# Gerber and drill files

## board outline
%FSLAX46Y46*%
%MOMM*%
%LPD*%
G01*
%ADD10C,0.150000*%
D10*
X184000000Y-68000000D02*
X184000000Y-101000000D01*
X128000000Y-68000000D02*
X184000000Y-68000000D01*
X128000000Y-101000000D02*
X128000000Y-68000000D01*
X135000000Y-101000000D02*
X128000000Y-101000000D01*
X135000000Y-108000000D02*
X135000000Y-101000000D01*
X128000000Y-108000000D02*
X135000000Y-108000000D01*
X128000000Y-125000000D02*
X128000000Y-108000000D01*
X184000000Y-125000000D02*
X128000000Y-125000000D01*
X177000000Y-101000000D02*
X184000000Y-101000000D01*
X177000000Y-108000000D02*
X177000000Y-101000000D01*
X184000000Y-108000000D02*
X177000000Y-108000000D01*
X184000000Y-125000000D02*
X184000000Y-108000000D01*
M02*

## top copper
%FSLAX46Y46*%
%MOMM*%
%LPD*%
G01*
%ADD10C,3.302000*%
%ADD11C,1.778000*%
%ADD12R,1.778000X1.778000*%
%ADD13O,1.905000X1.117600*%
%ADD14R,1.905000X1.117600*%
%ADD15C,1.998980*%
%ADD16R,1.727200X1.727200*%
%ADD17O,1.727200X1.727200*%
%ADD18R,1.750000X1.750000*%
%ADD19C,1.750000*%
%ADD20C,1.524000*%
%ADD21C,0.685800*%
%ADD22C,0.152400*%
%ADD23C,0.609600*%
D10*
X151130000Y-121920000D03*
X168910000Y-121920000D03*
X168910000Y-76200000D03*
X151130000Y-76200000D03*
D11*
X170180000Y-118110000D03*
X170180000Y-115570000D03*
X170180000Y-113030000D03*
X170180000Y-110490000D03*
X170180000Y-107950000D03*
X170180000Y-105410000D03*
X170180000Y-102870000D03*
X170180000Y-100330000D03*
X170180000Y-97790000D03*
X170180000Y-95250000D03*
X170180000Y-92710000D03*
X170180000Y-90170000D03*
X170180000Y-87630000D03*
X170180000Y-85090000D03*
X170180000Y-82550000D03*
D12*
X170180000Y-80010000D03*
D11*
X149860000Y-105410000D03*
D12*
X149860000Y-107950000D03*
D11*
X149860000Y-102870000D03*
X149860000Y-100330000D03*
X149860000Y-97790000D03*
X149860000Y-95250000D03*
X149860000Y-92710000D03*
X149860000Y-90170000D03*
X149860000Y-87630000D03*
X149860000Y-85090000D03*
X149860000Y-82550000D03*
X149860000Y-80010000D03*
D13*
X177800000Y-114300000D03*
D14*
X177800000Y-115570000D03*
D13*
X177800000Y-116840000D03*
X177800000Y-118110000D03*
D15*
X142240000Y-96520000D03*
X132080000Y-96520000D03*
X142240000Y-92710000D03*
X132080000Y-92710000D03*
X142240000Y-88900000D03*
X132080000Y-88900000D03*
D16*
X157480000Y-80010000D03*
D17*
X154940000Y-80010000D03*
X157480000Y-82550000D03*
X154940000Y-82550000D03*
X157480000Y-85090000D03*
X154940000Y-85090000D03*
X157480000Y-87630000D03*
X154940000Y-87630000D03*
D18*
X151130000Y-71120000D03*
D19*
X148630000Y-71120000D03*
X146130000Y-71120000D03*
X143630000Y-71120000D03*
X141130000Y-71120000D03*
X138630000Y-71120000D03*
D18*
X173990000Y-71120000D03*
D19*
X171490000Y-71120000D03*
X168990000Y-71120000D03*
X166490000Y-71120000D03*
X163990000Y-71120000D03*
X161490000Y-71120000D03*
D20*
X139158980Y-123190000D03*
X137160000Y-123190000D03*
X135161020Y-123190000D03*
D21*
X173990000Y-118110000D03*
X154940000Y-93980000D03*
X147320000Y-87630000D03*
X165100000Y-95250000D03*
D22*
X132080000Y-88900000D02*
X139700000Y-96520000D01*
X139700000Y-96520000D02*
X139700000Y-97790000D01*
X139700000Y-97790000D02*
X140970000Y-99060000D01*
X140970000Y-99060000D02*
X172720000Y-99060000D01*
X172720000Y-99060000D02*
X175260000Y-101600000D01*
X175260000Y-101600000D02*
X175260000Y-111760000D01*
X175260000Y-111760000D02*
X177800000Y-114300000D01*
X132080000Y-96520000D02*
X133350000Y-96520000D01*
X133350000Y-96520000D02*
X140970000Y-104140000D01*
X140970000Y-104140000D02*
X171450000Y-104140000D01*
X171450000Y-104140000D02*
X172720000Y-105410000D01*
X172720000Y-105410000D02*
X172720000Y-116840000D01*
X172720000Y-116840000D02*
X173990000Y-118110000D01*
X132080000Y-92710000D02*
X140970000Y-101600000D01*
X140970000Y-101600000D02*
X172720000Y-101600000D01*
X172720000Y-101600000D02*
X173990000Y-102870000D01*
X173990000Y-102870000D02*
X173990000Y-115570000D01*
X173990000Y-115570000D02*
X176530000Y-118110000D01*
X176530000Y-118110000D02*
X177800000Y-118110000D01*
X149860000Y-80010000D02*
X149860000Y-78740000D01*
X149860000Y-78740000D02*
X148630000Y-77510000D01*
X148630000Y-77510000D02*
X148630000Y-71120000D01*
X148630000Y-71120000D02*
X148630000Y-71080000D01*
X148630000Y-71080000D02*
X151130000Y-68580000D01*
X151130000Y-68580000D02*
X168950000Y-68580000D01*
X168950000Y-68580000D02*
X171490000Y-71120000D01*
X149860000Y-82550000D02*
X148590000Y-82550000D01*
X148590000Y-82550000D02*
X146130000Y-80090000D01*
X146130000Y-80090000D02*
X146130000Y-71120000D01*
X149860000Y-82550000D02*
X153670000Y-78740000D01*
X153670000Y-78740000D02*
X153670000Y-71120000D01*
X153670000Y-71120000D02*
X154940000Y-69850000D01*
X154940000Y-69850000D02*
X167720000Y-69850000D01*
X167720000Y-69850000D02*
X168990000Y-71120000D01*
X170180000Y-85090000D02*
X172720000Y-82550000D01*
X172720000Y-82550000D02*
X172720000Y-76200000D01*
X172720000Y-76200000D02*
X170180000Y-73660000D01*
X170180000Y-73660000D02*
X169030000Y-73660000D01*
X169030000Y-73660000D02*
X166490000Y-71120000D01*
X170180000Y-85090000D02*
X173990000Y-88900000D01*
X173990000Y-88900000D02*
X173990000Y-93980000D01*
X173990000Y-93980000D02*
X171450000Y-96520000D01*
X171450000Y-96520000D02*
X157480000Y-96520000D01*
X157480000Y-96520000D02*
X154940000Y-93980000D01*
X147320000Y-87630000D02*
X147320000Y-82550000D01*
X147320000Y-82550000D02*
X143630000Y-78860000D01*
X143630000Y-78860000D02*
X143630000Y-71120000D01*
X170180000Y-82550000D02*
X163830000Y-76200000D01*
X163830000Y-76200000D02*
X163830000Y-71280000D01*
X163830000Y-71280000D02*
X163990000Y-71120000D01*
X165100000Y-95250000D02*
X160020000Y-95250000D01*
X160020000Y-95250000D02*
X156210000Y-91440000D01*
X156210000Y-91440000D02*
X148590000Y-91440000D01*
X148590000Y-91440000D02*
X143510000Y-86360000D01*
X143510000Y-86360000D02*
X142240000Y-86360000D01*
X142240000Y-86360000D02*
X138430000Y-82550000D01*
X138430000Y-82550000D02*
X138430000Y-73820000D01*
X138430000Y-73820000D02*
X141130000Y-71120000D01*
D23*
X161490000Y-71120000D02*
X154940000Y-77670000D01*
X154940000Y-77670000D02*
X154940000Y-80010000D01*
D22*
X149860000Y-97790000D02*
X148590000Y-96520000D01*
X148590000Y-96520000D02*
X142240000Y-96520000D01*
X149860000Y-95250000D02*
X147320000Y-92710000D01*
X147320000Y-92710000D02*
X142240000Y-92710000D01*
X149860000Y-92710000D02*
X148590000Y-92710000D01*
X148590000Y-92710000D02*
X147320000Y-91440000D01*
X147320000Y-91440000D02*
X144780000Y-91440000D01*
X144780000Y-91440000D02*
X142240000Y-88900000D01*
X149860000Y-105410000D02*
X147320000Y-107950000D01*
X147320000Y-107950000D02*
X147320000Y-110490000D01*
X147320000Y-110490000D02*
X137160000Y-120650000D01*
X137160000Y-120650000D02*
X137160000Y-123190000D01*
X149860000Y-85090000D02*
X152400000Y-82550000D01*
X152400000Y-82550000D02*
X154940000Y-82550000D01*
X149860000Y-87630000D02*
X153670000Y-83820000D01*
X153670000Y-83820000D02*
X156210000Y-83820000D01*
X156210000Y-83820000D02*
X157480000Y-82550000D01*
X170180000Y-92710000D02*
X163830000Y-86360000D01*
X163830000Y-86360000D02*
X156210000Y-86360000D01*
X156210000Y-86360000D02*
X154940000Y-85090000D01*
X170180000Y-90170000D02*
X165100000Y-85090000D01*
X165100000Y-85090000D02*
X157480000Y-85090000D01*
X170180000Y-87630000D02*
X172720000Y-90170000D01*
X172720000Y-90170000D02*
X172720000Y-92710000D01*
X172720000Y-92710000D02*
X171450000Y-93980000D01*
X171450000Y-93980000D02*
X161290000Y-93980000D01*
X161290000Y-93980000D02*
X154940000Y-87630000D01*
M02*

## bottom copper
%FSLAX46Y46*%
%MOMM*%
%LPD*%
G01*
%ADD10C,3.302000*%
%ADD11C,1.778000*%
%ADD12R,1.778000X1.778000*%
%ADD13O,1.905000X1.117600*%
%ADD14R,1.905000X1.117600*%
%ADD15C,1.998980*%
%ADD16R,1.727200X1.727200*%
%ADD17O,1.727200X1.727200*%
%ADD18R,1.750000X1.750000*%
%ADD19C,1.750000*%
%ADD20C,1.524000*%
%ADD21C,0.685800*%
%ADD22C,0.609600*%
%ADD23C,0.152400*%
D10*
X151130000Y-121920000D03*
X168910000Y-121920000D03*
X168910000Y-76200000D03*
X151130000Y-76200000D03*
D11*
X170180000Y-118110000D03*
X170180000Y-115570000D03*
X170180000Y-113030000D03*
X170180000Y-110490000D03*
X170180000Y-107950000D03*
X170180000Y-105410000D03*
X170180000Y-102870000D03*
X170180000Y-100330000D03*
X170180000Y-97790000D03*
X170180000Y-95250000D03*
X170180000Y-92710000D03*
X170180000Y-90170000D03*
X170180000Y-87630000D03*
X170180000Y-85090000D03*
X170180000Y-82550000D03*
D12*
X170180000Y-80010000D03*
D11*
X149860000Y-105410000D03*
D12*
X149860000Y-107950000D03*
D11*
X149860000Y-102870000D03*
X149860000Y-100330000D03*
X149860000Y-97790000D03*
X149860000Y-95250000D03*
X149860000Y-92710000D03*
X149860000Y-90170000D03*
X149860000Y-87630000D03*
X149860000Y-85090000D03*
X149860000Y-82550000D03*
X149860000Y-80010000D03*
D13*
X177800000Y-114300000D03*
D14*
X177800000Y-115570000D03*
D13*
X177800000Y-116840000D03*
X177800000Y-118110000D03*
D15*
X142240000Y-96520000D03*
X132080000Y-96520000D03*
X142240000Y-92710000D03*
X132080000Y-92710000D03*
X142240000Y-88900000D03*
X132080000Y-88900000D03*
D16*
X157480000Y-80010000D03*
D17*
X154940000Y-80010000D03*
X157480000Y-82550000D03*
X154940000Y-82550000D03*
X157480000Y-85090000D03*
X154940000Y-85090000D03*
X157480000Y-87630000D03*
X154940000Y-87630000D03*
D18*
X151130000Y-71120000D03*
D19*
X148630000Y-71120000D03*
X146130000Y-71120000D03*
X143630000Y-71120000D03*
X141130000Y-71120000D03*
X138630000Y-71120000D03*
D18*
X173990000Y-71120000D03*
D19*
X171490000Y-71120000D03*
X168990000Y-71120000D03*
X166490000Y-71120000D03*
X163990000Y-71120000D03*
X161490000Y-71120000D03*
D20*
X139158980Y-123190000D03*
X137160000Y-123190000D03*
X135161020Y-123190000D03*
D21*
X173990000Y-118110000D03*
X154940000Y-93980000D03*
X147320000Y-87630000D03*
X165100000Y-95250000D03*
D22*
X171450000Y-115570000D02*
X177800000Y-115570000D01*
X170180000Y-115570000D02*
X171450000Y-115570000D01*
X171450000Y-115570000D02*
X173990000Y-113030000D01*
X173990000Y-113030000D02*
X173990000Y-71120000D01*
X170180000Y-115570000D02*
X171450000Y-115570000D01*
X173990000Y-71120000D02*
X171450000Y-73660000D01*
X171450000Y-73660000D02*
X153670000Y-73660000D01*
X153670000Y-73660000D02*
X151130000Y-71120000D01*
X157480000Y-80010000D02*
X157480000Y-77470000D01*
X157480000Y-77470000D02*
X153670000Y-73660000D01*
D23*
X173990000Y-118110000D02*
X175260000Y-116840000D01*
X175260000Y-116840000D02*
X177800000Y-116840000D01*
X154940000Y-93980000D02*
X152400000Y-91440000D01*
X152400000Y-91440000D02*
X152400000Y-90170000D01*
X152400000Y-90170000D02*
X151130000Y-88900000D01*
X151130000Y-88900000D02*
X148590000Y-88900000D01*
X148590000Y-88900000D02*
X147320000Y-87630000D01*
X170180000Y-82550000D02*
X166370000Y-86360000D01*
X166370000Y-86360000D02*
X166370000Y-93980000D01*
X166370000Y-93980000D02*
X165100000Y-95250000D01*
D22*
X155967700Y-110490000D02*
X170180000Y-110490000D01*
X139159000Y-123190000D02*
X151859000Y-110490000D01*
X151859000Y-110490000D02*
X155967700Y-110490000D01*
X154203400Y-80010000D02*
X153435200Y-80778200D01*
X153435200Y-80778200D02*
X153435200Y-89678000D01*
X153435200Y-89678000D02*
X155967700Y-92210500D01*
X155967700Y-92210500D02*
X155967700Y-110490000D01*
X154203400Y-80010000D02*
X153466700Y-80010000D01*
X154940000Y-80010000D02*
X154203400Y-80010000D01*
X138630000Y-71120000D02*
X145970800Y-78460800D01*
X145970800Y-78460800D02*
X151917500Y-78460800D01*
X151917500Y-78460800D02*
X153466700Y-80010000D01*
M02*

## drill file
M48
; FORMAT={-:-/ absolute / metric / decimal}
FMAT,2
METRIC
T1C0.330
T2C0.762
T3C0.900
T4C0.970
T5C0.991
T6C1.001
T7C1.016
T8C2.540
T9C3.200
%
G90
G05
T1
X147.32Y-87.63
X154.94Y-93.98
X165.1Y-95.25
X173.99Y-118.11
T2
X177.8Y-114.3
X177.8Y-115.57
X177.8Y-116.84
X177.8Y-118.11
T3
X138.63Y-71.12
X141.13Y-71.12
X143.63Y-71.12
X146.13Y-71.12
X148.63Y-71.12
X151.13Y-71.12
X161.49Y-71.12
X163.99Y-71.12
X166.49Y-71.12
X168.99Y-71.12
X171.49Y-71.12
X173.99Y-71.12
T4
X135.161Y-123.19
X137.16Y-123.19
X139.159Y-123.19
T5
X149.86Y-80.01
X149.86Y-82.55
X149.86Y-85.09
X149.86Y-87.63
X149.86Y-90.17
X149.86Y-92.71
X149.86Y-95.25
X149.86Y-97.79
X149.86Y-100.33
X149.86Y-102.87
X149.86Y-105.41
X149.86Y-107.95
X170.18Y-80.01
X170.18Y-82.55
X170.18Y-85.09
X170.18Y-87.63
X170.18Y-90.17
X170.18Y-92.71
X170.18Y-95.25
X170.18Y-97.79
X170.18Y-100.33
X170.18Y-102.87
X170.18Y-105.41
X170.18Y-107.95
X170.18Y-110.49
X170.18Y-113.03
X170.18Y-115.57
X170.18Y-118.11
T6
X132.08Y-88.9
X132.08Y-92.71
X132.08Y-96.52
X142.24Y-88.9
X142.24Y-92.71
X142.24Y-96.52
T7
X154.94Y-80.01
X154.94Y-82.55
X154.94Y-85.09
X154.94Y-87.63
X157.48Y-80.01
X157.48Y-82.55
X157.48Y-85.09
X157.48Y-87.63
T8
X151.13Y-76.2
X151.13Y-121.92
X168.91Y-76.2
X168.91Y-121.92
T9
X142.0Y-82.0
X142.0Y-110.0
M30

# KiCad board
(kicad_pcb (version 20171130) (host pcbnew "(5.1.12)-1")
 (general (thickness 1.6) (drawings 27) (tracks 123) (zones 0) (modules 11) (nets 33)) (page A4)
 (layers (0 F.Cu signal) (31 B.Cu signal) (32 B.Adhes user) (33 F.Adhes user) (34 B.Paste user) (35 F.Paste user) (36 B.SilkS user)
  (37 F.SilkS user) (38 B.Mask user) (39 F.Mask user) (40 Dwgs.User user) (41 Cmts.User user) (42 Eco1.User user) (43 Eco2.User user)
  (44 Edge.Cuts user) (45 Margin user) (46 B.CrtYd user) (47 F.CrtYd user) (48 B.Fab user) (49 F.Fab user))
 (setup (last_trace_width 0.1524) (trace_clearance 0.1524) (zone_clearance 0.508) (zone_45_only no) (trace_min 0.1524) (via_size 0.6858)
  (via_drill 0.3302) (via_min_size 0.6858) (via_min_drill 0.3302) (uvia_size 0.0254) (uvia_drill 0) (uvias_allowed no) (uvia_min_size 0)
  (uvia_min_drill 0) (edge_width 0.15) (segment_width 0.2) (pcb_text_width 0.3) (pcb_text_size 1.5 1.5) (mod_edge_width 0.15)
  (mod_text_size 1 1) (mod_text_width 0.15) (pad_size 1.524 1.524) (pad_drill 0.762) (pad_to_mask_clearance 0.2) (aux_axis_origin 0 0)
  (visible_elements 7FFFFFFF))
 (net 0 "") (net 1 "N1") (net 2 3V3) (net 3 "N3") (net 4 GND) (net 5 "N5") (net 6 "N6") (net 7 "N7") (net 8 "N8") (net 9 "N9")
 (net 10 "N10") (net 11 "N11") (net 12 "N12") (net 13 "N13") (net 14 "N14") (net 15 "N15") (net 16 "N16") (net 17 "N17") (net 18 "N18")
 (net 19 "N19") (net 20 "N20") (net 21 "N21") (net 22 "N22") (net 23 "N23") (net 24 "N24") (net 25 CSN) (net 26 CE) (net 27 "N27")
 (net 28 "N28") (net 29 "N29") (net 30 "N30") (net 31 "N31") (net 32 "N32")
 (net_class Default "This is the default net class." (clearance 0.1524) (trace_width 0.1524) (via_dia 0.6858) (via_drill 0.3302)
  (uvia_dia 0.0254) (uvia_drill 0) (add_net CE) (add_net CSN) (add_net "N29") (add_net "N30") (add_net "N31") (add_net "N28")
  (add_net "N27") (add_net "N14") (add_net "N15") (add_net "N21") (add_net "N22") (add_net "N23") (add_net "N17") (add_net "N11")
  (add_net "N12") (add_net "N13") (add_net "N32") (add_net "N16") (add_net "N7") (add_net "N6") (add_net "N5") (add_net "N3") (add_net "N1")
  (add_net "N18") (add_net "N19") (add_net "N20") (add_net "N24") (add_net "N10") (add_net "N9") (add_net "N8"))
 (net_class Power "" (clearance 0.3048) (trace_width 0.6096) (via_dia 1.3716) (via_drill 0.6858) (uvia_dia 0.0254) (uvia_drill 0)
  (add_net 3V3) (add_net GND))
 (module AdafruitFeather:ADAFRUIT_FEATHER (layer F.Cu) (at 160.02 99.06 90)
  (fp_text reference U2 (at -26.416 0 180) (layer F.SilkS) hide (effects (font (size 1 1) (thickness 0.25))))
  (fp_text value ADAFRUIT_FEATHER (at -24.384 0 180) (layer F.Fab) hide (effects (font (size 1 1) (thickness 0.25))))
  (pad "" thru_hole circle (at -22.86 -8.89 90) (size 3.302 3.302) (drill 2.54) (layers *.Cu *.Mask F.SilkS))
  (pad "" thru_hole circle (at -22.86 8.89 90) (size 3.302 3.302) (drill 2.54) (layers *.Cu *.Mask F.SilkS))
  (pad "" thru_hole circle (at 22.86 8.89 90) (size 3.302 3.302) (drill 2.54) (layers *.Cu *.Mask F.SilkS))
  (pad "" thru_hole circle (at 22.86 -8.89 90) (size 3.302 3.302) (drill 2.54) (layers *.Cu *.Mask F.SilkS))
  (pad 16 thru_hole circle (at -19.05 10.16 90) (size 1.778 1.778) (drill 0.9906) (layers *.Cu *.Mask F.SilkS) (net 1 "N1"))
  (pad 15 thru_hole circle (at -16.51 10.16 90) (size 1.778 1.778) (drill 0.9906) (layers *.Cu *.Mask F.SilkS) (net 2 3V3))
  (pad 14 thru_hole circle (at -13.97 10.16 90) (size 1.778 1.778) (drill 0.9906) (layers *.Cu *.Mask F.SilkS) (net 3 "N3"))
  (pad 13 thru_hole circle (at -11.43 10.16 90) (size 1.778 1.778) (drill 0.9906) (layers *.Cu *.Mask F.SilkS) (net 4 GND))
  (pad 12 thru_hole circle (at -8.89 10.16 90) (size 1.778 1.778) (drill 0.9906) (layers *.Cu *.Mask F.SilkS) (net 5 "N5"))
  (pad 11 thru_hole circle (at -6.35 10.16 90) (size 1.778 1.778) (drill 0.9906) (layers *.Cu *.Mask F.SilkS) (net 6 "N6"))
  (pad 10 thru_hole circle (at -3.81 10.16 90) (size 1.778 1.778) (drill 0.9906) (layers *.Cu *.Mask F.SilkS) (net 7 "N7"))
  (pad 9 thru_hole circle (at -1.27 10.16 90) (size 1.778 1.778) (drill 0.9906) (layers *.Cu *.Mask F.SilkS) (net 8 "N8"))
  (pad 8 thru_hole circle (at 1.27 10.16 90) (size 1.778 1.778) (drill 0.9906) (layers *.Cu *.Mask F.SilkS) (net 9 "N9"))
  (pad 7 thru_hole circle (at 3.81 10.16 90) (size 1.778 1.778) (drill 0.9906) (layers *.Cu *.Mask F.SilkS) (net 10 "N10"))
  (pad 6 thru_hole circle (at 6.35 10.16 90) (size 1.778 1.778) (drill 0.9906) (layers *.Cu *.Mask F.SilkS) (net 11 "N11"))
  (pad 5 thru_hole circle (at 8.89 10.16 90) (size 1.778 1.778) (drill 0.9906) (layers *.Cu *.Mask F.SilkS) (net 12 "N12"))
  (pad 4 thru_hole circle (at 11.43 10.16 90) (size 1.778 1.778) (drill 0.9906) (layers *.Cu *.Mask F.SilkS) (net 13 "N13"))
  (pad 3 thru_hole circle (at 13.97 10.16 90) (size 1.778 1.778) (drill 0.9906) (layers *.Cu *.Mask F.SilkS) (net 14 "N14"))
  (pad 2 thru_hole circle (at 16.51 10.16 90) (size 1.778 1.778) (drill 0.9906) (layers *.Cu *.Mask F.SilkS) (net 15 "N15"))
  (pad 1 thru_hole rect (at 19.05 10.16 90) (size 1.778 1.778) (drill 0.9906) (layers *.Cu *.Mask F.SilkS) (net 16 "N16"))
  (pad 18 thru_hole circle (at -6.35 -10.16 90) (size 1.778 1.778) (drill 0.9906) (layers *.Cu *.Mask F.SilkS) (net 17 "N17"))
  (pad 17 thru_hole rect (at -8.89 -10.16 90) (size 1.778 1.778) (drill 0.9906) (layers *.Cu *.Mask F.SilkS) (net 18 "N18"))
  (pad 19 thru_hole circle (at -3.81 -10.16 90) (size 1.778 1.778) (drill 0.9906) (layers *.Cu *.Mask F.SilkS) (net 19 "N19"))
  (pad 20 thru_hole circle (at -1.27 -10.16 90) (size 1.778 1.778) (drill 0.9906) (layers *.Cu *.Mask F.SilkS) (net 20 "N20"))
  (pad 21 thru_hole circle (at 1.27 -10.16 90) (size 1.778 1.778) (drill 0.9906) (layers *.Cu *.Mask F.SilkS) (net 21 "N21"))
  (pad 22 thru_hole circle (at 3.81 -10.16 90) (size 1.778 1.778) (drill 0.9906) (layers *.Cu *.Mask F.SilkS) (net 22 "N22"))
  (pad 23 thru_hole circle (at 6.35 -10.16 90) (size 1.778 1.778) (drill 0.9906) (layers *.Cu *.Mask F.SilkS) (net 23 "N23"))
  (pad 24 thru_hole circle (at 8.89 -10.16 90) (size 1.778 1.778) (drill 0.9906) (layers *.Cu *.Mask F.SilkS) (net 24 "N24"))
  (pad 25 thru_hole circle (at 11.43 -10.16 90) (size 1.778 1.778) (drill 0.9906) (layers *.Cu *.Mask F.SilkS) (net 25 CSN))
  (pad 26 thru_hole circle (at 13.97 -10.16 90) (size 1.778 1.778) (drill 0.9906) (layers *.Cu *.Mask F.SilkS) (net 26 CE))
  (pad 27 thru_hole circle (at 16.51 -10.16 90) (size 1.778 1.778) (drill 0.9906) (layers *.Cu *.Mask F.SilkS) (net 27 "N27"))
  (pad 28 thru_hole circle (at 19.05 -10.16 90) (size 1.778 1.778) (drill 0.9906) (layers *.Cu *.Mask F.SilkS) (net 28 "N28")))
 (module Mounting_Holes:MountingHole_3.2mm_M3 (layer F.Cu) (at 142 110)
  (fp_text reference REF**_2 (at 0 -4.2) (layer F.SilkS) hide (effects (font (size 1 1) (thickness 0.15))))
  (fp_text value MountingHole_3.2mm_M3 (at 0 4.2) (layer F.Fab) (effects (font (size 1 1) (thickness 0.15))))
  (pad 1 np_thru_hole circle (at 0 0) (size 3.2 3.2) (drill 3.2) (layers *.Cu *.Mask)))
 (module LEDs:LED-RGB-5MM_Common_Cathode (layer F.Cu) (at 177.8 114.3)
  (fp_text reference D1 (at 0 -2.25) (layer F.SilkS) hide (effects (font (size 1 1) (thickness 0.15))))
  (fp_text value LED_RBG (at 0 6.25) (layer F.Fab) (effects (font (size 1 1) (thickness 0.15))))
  (pad 1 thru_hole oval (at 0 0) (size 1.905 1.1176) (drill 0.762) (layers *.Cu *.Mask) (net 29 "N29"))
  (pad 2 thru_hole rect (at 0 1.27) (size 1.905 1.1176) (drill 0.762) (layers *.Cu *.Mask) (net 2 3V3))
  (pad 3 thru_hole oval (at 0 2.54) (size 1.905 1.1176) (drill 0.762) (layers *.Cu *.Mask) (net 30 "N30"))
  (pad 4 thru_hole oval (at 0 3.81) (size 1.905 1.1176) (drill 0.762) (layers *.Cu *.Mask) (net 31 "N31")))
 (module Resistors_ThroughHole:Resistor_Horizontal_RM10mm (layer F.Cu) (at 142.24 96.52 180)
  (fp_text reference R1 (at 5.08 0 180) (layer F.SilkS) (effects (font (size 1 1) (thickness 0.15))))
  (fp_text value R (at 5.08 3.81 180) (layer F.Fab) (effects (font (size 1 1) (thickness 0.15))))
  (pad 1 thru_hole circle (at 0 0 180) (size 1.99898 1.99898) (drill 1.00076) (layers *.Cu *.SilkS *.Mask) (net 21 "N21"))
  (pad 2 thru_hole circle (at 10.16 0 180) (size 1.99898 1.99898) (drill 1.00076) (layers *.Cu *.SilkS *.Mask) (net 30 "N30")))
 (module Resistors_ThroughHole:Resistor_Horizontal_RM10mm (layer F.Cu) (at 142.24 92.71 180)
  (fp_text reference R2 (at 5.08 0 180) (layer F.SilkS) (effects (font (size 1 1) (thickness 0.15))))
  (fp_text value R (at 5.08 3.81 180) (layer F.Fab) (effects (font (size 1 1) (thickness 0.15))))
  (pad 1 thru_hole circle (at 0 0 180) (size 1.99898 1.99898) (drill 1.00076) (layers *.Cu *.SilkS *.Mask) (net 22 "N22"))
  (pad 2 thru_hole circle (at 10.16 0 180) (size 1.99898 1.99898) (drill 1.00076) (layers *.Cu *.SilkS *.Mask) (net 31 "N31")))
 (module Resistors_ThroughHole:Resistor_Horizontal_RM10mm (layer F.Cu) (at 142.24 88.9 180)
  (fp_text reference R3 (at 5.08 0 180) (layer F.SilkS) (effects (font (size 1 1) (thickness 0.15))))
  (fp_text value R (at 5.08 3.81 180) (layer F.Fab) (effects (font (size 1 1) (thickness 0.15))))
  (pad 1 thru_hole circle (at 0 0 180) (size 1.99898 1.99898) (drill 1.00076) (layers *.Cu *.SilkS *.Mask) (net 23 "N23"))
  (pad 2 thru_hole circle (at 10.16 0 180) (size 1.99898 1.99898) (drill 1.00076) (layers *.Cu *.SilkS *.Mask) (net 29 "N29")))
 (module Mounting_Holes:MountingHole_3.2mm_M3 (layer F.Cu) (at 142 82)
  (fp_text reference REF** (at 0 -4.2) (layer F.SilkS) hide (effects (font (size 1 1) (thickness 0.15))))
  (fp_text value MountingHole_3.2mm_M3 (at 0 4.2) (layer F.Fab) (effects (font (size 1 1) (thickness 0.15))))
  (pad 1 np_thru_hole circle (at 0 0) (size 3.2 3.2) (drill 3.2) (layers *.Cu *.Mask)))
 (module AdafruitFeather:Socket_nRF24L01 (layer F.Cu) (at 157.48 80.01 270)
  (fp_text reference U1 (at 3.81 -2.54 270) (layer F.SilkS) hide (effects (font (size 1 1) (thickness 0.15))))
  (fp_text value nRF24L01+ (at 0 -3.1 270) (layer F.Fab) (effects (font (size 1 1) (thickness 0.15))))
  (pad 2 thru_hole rect (at 0 0 270) (size 1.7272 1.7272) (drill 1.016) (layers *.Cu *.Mask F.SilkS) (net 2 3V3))
  (pad 1 thru_hole oval (at 0 2.54 270) (size 1.7272 1.7272) (drill 1.016) (layers *.Cu *.Mask F.SilkS) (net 4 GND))
  (pad 4 thru_hole oval (at 2.54 0 270) (size 1.7272 1.7272) (drill 1.016) (layers *.Cu *.Mask F.SilkS) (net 25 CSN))
  (pad 3 thru_hole oval (at 2.54 2.54 270) (size 1.7272 1.7272) (drill 1.016) (layers *.Cu *.Mask F.SilkS) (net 26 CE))
  (pad 6 thru_hole oval (at 5.08 0 270) (size 1.7272 1.7272) (drill 1.016) (layers *.Cu *.Mask F.SilkS) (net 12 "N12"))
  (pad 5 thru_hole oval (at 5.08 2.54 270) (size 1.7272 1.7272) (drill 1.016) (layers *.Cu *.Mask F.SilkS) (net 11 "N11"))
  (pad 8 thru_hole oval (at 7.62 0 270) (size 1.7272 1.7272) (drill 1.016) (layers *.Cu *.Mask F.SilkS) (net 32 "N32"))
  (pad 7 thru_hole oval (at 7.62 2.54 270) (size 1.7272 1.7272) (drill 1.016) (layers *.Cu *.Mask F.SilkS) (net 13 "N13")))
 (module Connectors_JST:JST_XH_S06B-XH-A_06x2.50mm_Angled (layer F.Cu) (at 151.13 71.12 180)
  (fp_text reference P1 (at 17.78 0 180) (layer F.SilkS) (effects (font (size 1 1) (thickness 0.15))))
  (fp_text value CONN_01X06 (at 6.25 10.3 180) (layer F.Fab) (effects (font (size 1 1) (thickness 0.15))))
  (pad 1 thru_hole rect (at 0 0 180) (size 1.75 1.75) (drill 0.9) (layers *.Cu *.Mask) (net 2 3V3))
  (pad 2 thru_hole circle (at 2.5 0 180) (size 1.75 1.75) (drill 0.9) (layers *.Cu *.Mask) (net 28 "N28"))
  (pad 3 thru_hole circle (at 5 0 180) (size 1.75 1.75) (drill 0.9) (layers *.Cu *.Mask) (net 27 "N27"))
  (pad 4 thru_hole circle (at 7.5 0 180) (size 1.75 1.75) (drill 0.9) (layers *.Cu *.Mask) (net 14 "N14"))
  (pad 5 thru_hole circle (at 10 0 180) (size 1.75 1.75) (drill 0.9) (layers *.Cu *.Mask) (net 15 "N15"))
  (pad 6 thru_hole circle (at 12.5 0 180) (size 1.75 1.75) (drill 0.9) (layers *.Cu *.Mask) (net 4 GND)))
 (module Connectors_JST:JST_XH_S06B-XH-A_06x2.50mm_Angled (layer F.Cu) (at 173.99 71.12 180)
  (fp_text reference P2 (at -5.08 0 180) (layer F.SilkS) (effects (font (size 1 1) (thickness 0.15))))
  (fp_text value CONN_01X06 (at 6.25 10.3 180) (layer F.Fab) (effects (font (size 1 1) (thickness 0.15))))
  (pad 1 thru_hole rect (at 0 0 180) (size 1.75 1.75) (drill 0.9) (layers *.Cu *.Mask) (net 2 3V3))
  (pad 2 thru_hole circle (at 2.5 0 180) (size 1.75 1.75) (drill 0.9) (layers *.Cu *.Mask) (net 28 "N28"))
  (pad 3 thru_hole circle (at 5 0 180) (size 1.75 1.75) (drill 0.9) (layers *.Cu *.Mask) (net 27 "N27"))
  (pad 4 thru_hole circle (at 7.5 0 180) (size 1.75 1.75) (drill 0.9) (layers *.Cu *.Mask) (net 14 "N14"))
  (pad 5 thru_hole circle (at 10 0 180) (size 1.75 1.75) (drill 0.9) (layers *.Cu *.Mask) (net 15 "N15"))
  (pad 6 thru_hole circle (at 12.5 0 180) (size 1.75 1.75) (drill 0.9) (layers *.Cu *.Mask) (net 4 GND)))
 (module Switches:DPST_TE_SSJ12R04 (layer F.Cu) (at 137.16 123.19 180)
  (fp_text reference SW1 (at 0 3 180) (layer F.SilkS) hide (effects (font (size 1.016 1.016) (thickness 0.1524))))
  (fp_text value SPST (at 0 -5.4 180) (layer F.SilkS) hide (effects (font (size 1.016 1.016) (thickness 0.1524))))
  (pad 1 thru_hole circle (at -1.99898 0 180) (size 1.524 1.524) (drill 0.97028) (layers *.Cu *.Mask F.SilkS) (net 4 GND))
  (pad 2 thru_hole circle (at 0 0 180) (size 1.524 1.524) (drill 0.97028) (layers *.Cu *.Mask F.SilkS) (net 17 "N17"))
  (pad 3 thru_hole circle (at 1.99898 0 180) (size 1.524 1.524) (drill 0.97028) (layers *.Cu *.Mask F.SilkS)))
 (gr_line (start 184 68) (end 184 101) (angle 90) (layer Edge.Cuts) (width 0.15))
 (gr_line (start 128 68) (end 184 68) (angle 90) (layer Edge.Cuts) (width 0.15))
 (gr_line (start 128 101) (end 128 68) (angle 90) (layer Edge.Cuts) (width 0.15))
 (gr_line (start 135 101) (end 128 101) (angle 90) (layer Edge.Cuts) (width 0.15))
 (gr_line (start 135 108) (end 135 101) (angle 90) (layer Edge.Cuts) (width 0.15))
 (gr_line (start 128 108) (end 135 108) (angle 90) (layer Edge.Cuts) (width 0.15))
 (gr_line (start 128 125) (end 128 108) (angle 90) (layer Edge.Cuts) (width 0.15))
 (gr_line (start 184 125) (end 128 125) (angle 90) (layer Edge.Cuts) (width 0.15))
 (gr_line (start 177 101) (end 184 101) (angle 90) (layer Edge.Cuts) (width 0.15))
 (gr_line (start 177 108) (end 177 101) (angle 90) (layer Edge.Cuts) (width 0.15))
 (gr_line (start 184 108) (end 177 108) (angle 90) (layer Edge.Cuts) (width 0.15))
 (gr_line (start 184 125) (end 184 108) (angle 90) (layer Edge.Cuts) (width 0.15))
 (segment (start 132.08 88.9) (end 139.7 96.52) (width 0.1524) (layer F.Cu) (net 29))
 (segment (start 139.7 96.52) (end 139.7 97.79) (width 0.1524) (layer F.Cu) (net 29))
 (segment (start 139.7 97.79) (end 140.97 99.06) (width 0.1524) (layer F.Cu) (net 29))
 (segment (start 140.97 99.06) (end 172.72 99.06) (width 0.1524) (layer F.Cu) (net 29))
 (segment (start 172.72 99.06) (end 175.26 101.6) (width 0.1524) (layer F.Cu) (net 29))
 (segment (start 175.26 101.6) (end 175.26 111.76) (width 0.1524) (layer F.Cu) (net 29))
 (segment (start 175.26 111.76) (end 177.8 114.3) (width 0.1524) (layer F.Cu) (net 29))
 (segment (start 171.45 115.57) (end 177.8 115.57) (width 0.6096) (layer B.Cu) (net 2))
 (segment (start 170.18 115.57) (end 171.45 115.57) (width 0.6096) (layer B.Cu) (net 2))
 (segment (start 171.45 115.57) (end 173.99 113.03) (width 0.6096) (layer B.Cu) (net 2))
 (segment (start 173.99 113.03) (end 173.99 71.12) (width 0.6096) (layer B.Cu) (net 2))
 (segment (start 170.18 115.57) (end 171.45 115.57) (width 0.6096) (layer B.Cu) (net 2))
 (segment (start 173.99 71.12) (end 171.45 73.66) (width 0.6096) (layer B.Cu) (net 2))
 (segment (start 171.45 73.66) (end 153.67 73.66) (width 0.6096) (layer B.Cu) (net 2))
 (segment (start 153.67 73.66) (end 151.13 71.12) (width 0.6096) (layer B.Cu) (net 2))
 (segment (start 157.48 80.01) (end 157.48 77.47) (width 0.6096) (layer B.Cu) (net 2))
 (segment (start 157.48 77.47) (end 153.67 73.66) (width 0.6096) (layer B.Cu) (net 2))
 (segment (start 132.08 96.52) (end 133.35 96.52) (width 0.1524) (layer F.Cu) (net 30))
 (segment (start 133.35 96.52) (end 140.97 104.14) (width 0.1524) (layer F.Cu) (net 30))
 (segment (start 140.97 104.14) (end 171.45 104.14) (width 0.1524) (layer F.Cu) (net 30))
 (segment (start 171.45 104.14) (end 172.72 105.41) (width 0.1524) (layer F.Cu) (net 30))
 (segment (start 172.72 105.41) (end 172.72 116.84) (width 0.1524) (layer F.Cu) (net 30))
 (segment (start 172.72 116.84) (end 173.99 118.11) (width 0.1524) (layer F.Cu) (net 30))
 (segment (start 173.99 118.11) (end 175.26 116.84) (width 0.1524) (layer B.Cu) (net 30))
 (segment (start 175.26 116.84) (end 177.8 116.84) (width 0.1524) (layer B.Cu) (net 30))
 (via (at 173.99 118.11) (size 0.6858) (layers F.Cu B.Cu) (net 30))
 (segment (start 132.08 92.71) (end 140.97 101.6) (width 0.1524) (layer F.Cu) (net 31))
 (segment (start 140.97 101.6) (end 172.72 101.6) (width 0.1524) (layer F.Cu) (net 31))
 (segment (start 172.72 101.6) (end 173.99 102.87) (width 0.1524) (layer F.Cu) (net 31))
 (segment (start 173.99 102.87) (end 173.99 115.57) (width 0.1524) (layer F.Cu) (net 31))
 (segment (start 173.99 115.57) (end 176.53 118.11) (width 0.1524) (layer F.Cu) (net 31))
 (segment (start 176.53 118.11) (end 177.8 118.11) (width 0.1524) (layer F.Cu) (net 31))
 (segment (start 149.86 80.01) (end 149.86 78.74) (width 0.1524) (layer F.Cu) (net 28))
 (segment (start 149.86 78.74) (end 148.63 77.51) (width 0.1524) (layer F.Cu) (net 28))
 (segment (start 148.63 77.51) (end 148.63 71.12) (width 0.1524) (layer F.Cu) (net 28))
 (segment (start 148.63 71.12) (end 148.63 71.08) (width 0.1524) (layer F.Cu) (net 28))
 (segment (start 148.63 71.08) (end 151.13 68.58) (width 0.1524) (layer F.Cu) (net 28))
 (segment (start 151.13 68.58) (end 168.95 68.58) (width 0.1524) (layer F.Cu) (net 28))
 (segment (start 168.95 68.58) (end 171.49 71.12) (width 0.1524) (layer F.Cu) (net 28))
 (segment (start 149.86 82.55) (end 148.59 82.55) (width 0.1524) (layer F.Cu) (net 27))
 (segment (start 148.59 82.55) (end 146.13 80.09) (width 0.1524) (layer F.Cu) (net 27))
 (segment (start 146.13 80.09) (end 146.13 71.12) (width 0.1524) (layer F.Cu) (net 27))
 (segment (start 149.86 82.55) (end 153.67 78.74) (width 0.1524) (layer F.Cu) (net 27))
 (segment (start 153.67 78.74) (end 153.67 71.12) (width 0.1524) (layer F.Cu) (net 27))
 (segment (start 153.67 71.12) (end 154.94 69.85) (width 0.1524) (layer F.Cu) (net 27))
 (segment (start 154.94 69.85) (end 167.72 69.85) (width 0.1524) (layer F.Cu) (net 27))
 (segment (start 167.72 69.85) (end 168.99 71.12) (width 0.1524) (layer F.Cu) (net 27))
 (segment (start 170.18 85.09) (end 172.72 82.55) (width 0.1524) (layer F.Cu) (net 14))
 (segment (start 172.72 82.55) (end 172.72 76.2) (width 0.1524) (layer F.Cu) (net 14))
 (segment (start 172.72 76.2) (end 170.18 73.66) (width 0.1524) (layer F.Cu) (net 14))
 (segment (start 170.18 73.66) (end 169.03 73.66) (width 0.1524) (layer F.Cu) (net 14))
 (segment (start 169.03 73.66) (end 166.49 71.12) (width 0.1524) (layer F.Cu) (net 14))
 (segment (start 170.18 85.09) (end 173.99 88.9) (width 0.1524) (layer F.Cu) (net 14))
 (segment (start 173.99 88.9) (end 173.99 93.98) (width 0.1524) (layer F.Cu) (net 14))
 (segment (start 173.99 93.98) (end 171.45 96.52) (width 0.1524) (layer F.Cu) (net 14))
 (segment (start 171.45 96.52) (end 157.48 96.52) (width 0.1524) (layer F.Cu) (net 14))
 (segment (start 157.48 96.52) (end 154.94 93.98) (width 0.1524) (layer F.Cu) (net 14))
 (segment (start 154.94 93.98) (end 152.4 91.44) (width 0.1524) (layer B.Cu) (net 14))
 (segment (start 152.4 91.44) (end 152.4 90.17) (width 0.1524) (layer B.Cu) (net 14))
 (segment (start 152.4 90.17) (end 151.13 88.9) (width 0.1524) (layer B.Cu) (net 14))
 (segment (start 151.13 88.9) (end 148.59 88.9) (width 0.1524) (layer B.Cu) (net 14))
 (segment (start 148.59 88.9) (end 147.32 87.63) (width 0.1524) (layer B.Cu) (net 14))
 (segment (start 147.32 87.63) (end 147.32 82.55) (width 0.1524) (layer F.Cu) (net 14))
 (segment (start 147.32 82.55) (end 143.63 78.86) (width 0.1524) (layer F.Cu) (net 14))
 (segment (start 143.63 78.86) (end 143.63 71.12) (width 0.1524) (layer F.Cu) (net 14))
 (via (at 154.94 93.98) (size 0.6858) (layers F.Cu B.Cu) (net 14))
 (via (at 147.32 87.63) (size 0.6858) (layers F.Cu B.Cu) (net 14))
 (segment (start 170.18 82.55) (end 163.83 76.2) (width 0.1524) (layer F.Cu) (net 15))
 (segment (start 163.83 76.2) (end 163.83 71.28) (width 0.1524) (layer F.Cu) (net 15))
 (segment (start 163.83 71.28) (end 163.99 71.12) (width 0.1524) (layer F.Cu) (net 15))
 (segment (start 170.18 82.55) (end 166.37 86.36) (width 0.1524) (layer B.Cu) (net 15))
 (segment (start 166.37 86.36) (end 166.37 93.98) (width 0.1524) (layer B.Cu) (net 15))
 (segment (start 166.37 93.98) (end 165.1 95.25) (width 0.1524) (layer B.Cu) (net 15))
 (segment (start 165.1 95.25) (end 160.02 95.25) (width 0.1524) (layer F.Cu) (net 15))
 (segment (start 160.02 95.25) (end 156.21 91.44) (width 0.1524) (layer F.Cu) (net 15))
 (segment (start 156.21 91.44) (end 148.59 91.44) (width 0.1524) (layer F.Cu) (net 15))
 (segment (start 148.59 91.44) (end 143.51 86.36) (width 0.1524) (layer F.Cu) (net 15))
 (segment (start 143.51 86.36) (end 142.24 86.36) (width 0.1524) (layer F.Cu) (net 15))
 (segment (start 142.24 86.36) (end 138.43 82.55) (width 0.1524) (layer F.Cu) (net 15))
 (segment (start 138.43 82.55) (end 138.43 73.82) (width 0.1524) (layer F.Cu) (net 15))
 (segment (start 138.43 73.82) (end 141.13 71.12) (width 0.1524) (layer F.Cu) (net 15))
 (via (at 165.1 95.25) (size 0.6858) (layers F.Cu B.Cu) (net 15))
 (segment (start 155.9677 110.49) (end 170.18 110.49) (width 0.6096) (layer B.Cu) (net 4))
 (segment (start 139.159 123.19) (end 151.859 110.49) (width 0.6096) (layer B.Cu) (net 4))
 (segment (start 151.859 110.49) (end 155.9677 110.49) (width 0.6096) (layer B.Cu) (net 4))
 (segment (start 154.2034 80.01) (end 153.4352 80.7782) (width 0.6096) (layer B.Cu) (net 4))
 (segment (start 153.4352 80.7782) (end 153.4352 89.678) (width 0.6096) (layer B.Cu) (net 4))
 (segment (start 153.4352 89.678) (end 155.9677 92.2105) (width 0.6096) (layer B.Cu) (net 4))
 (segment (start 155.9677 92.2105) (end 155.9677 110.49) (width 0.6096) (layer B.Cu) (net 4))
 (segment (start 154.2034 80.01) (end 153.4667 80.01) (width 0.6096) (layer B.Cu) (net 4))
 (segment (start 154.94 80.01) (end 154.2034 80.01) (width 0.6096) (layer B.Cu) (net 4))
 (segment (start 138.63 71.12) (end 145.9708 78.4608) (width 0.6096) (layer B.Cu) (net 4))
 (segment (start 145.9708 78.4608) (end 151.9175 78.4608) (width 0.6096) (layer B.Cu) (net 4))
 (segment (start 151.9175 78.4608) (end 153.4667 80.01) (width 0.6096) (layer B.Cu) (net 4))
 (segment (start 161.49 71.12) (end 154.94 77.67) (width 0.6096) (layer F.Cu) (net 4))
 (segment (start 154.94 77.67) (end 154.94 80.01) (width 0.6096) (layer F.Cu) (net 4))
 (segment (start 149.86 97.79) (end 148.59 96.52) (width 0.1524) (layer F.Cu) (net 21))
 (segment (start 148.59 96.52) (end 142.24 96.52) (width 0.1524) (layer F.Cu) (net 21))
 (segment (start 149.86 95.25) (end 147.32 92.71) (width 0.1524) (layer F.Cu) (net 22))
 (segment (start 147.32 92.71) (end 142.24 92.71) (width 0.1524) (layer F.Cu) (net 22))
 (segment (start 149.86 92.71) (end 148.59 92.71) (width 0.1524) (layer F.Cu) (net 23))
 (segment (start 148.59 92.71) (end 147.32 91.44) (width 0.1524) (layer F.Cu) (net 23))
 (segment (start 147.32 91.44) (end 144.78 91.44) (width 0.1524) (layer F.Cu) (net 23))
 (segment (start 144.78 91.44) (end 142.24 88.9) (width 0.1524) (layer F.Cu) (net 23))
 (segment (start 149.86 105.41) (end 147.32 107.95) (width 0.1524) (layer F.Cu) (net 17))
 (segment (start 147.32 107.95) (end 147.32 110.49) (width 0.1524) (layer F.Cu) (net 17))
 (segment (start 147.32 110.49) (end 137.16 120.65) (width 0.1524) (layer F.Cu) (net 17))
 (segment (start 137.16 120.65) (end 137.16 123.19) (width 0.1524) (layer F.Cu) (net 17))
 (segment (start 149.86 85.09) (end 152.4 82.55) (width 0.1524) (layer F.Cu) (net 26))
 (segment (start 152.4 82.55) (end 154.94 82.55) (width 0.1524) (layer F.Cu) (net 26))
 (segment (start 149.86 87.63) (end 153.67 83.82) (width 0.1524) (layer F.Cu) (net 25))
 (segment (start 153.67 83.82) (end 156.21 83.82) (width 0.1524) (layer F.Cu) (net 25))
 (segment (start 156.21 83.82) (end 157.48 82.55) (width 0.1524) (layer F.Cu) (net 25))
 (segment (start 170.18 92.71) (end 163.83 86.36) (width 0.1524) (layer F.Cu) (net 11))
 (segment (start 163.83 86.36) (end 156.21 86.36) (width 0.1524) (layer F.Cu) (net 11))
 (segment (start 156.21 86.36) (end 154.94 85.09) (width 0.1524) (layer F.Cu) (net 11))
 (segment (start 170.18 90.17) (end 165.1 85.09) (width 0.1524) (layer F.Cu) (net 12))
 (segment (start 165.1 85.09) (end 157.48 85.09) (width 0.1524) (layer F.Cu) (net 12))
 (segment (start 170.18 87.63) (end 172.72 90.17) (width 0.1524) (layer F.Cu) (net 13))
 (segment (start 172.72 90.17) (end 172.72 92.71) (width 0.1524) (layer F.Cu) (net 13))
 (segment (start 172.72 92.71) (end 171.45 93.98) (width 0.1524) (layer F.Cu) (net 13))
 (segment (start 171.45 93.98) (end 161.29 93.98) (width 0.1524) (layer F.Cu) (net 13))
 (segment (start 161.29 93.98) (end 154.94 87.63) (width 0.1524) (layer F.Cu) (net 13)))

